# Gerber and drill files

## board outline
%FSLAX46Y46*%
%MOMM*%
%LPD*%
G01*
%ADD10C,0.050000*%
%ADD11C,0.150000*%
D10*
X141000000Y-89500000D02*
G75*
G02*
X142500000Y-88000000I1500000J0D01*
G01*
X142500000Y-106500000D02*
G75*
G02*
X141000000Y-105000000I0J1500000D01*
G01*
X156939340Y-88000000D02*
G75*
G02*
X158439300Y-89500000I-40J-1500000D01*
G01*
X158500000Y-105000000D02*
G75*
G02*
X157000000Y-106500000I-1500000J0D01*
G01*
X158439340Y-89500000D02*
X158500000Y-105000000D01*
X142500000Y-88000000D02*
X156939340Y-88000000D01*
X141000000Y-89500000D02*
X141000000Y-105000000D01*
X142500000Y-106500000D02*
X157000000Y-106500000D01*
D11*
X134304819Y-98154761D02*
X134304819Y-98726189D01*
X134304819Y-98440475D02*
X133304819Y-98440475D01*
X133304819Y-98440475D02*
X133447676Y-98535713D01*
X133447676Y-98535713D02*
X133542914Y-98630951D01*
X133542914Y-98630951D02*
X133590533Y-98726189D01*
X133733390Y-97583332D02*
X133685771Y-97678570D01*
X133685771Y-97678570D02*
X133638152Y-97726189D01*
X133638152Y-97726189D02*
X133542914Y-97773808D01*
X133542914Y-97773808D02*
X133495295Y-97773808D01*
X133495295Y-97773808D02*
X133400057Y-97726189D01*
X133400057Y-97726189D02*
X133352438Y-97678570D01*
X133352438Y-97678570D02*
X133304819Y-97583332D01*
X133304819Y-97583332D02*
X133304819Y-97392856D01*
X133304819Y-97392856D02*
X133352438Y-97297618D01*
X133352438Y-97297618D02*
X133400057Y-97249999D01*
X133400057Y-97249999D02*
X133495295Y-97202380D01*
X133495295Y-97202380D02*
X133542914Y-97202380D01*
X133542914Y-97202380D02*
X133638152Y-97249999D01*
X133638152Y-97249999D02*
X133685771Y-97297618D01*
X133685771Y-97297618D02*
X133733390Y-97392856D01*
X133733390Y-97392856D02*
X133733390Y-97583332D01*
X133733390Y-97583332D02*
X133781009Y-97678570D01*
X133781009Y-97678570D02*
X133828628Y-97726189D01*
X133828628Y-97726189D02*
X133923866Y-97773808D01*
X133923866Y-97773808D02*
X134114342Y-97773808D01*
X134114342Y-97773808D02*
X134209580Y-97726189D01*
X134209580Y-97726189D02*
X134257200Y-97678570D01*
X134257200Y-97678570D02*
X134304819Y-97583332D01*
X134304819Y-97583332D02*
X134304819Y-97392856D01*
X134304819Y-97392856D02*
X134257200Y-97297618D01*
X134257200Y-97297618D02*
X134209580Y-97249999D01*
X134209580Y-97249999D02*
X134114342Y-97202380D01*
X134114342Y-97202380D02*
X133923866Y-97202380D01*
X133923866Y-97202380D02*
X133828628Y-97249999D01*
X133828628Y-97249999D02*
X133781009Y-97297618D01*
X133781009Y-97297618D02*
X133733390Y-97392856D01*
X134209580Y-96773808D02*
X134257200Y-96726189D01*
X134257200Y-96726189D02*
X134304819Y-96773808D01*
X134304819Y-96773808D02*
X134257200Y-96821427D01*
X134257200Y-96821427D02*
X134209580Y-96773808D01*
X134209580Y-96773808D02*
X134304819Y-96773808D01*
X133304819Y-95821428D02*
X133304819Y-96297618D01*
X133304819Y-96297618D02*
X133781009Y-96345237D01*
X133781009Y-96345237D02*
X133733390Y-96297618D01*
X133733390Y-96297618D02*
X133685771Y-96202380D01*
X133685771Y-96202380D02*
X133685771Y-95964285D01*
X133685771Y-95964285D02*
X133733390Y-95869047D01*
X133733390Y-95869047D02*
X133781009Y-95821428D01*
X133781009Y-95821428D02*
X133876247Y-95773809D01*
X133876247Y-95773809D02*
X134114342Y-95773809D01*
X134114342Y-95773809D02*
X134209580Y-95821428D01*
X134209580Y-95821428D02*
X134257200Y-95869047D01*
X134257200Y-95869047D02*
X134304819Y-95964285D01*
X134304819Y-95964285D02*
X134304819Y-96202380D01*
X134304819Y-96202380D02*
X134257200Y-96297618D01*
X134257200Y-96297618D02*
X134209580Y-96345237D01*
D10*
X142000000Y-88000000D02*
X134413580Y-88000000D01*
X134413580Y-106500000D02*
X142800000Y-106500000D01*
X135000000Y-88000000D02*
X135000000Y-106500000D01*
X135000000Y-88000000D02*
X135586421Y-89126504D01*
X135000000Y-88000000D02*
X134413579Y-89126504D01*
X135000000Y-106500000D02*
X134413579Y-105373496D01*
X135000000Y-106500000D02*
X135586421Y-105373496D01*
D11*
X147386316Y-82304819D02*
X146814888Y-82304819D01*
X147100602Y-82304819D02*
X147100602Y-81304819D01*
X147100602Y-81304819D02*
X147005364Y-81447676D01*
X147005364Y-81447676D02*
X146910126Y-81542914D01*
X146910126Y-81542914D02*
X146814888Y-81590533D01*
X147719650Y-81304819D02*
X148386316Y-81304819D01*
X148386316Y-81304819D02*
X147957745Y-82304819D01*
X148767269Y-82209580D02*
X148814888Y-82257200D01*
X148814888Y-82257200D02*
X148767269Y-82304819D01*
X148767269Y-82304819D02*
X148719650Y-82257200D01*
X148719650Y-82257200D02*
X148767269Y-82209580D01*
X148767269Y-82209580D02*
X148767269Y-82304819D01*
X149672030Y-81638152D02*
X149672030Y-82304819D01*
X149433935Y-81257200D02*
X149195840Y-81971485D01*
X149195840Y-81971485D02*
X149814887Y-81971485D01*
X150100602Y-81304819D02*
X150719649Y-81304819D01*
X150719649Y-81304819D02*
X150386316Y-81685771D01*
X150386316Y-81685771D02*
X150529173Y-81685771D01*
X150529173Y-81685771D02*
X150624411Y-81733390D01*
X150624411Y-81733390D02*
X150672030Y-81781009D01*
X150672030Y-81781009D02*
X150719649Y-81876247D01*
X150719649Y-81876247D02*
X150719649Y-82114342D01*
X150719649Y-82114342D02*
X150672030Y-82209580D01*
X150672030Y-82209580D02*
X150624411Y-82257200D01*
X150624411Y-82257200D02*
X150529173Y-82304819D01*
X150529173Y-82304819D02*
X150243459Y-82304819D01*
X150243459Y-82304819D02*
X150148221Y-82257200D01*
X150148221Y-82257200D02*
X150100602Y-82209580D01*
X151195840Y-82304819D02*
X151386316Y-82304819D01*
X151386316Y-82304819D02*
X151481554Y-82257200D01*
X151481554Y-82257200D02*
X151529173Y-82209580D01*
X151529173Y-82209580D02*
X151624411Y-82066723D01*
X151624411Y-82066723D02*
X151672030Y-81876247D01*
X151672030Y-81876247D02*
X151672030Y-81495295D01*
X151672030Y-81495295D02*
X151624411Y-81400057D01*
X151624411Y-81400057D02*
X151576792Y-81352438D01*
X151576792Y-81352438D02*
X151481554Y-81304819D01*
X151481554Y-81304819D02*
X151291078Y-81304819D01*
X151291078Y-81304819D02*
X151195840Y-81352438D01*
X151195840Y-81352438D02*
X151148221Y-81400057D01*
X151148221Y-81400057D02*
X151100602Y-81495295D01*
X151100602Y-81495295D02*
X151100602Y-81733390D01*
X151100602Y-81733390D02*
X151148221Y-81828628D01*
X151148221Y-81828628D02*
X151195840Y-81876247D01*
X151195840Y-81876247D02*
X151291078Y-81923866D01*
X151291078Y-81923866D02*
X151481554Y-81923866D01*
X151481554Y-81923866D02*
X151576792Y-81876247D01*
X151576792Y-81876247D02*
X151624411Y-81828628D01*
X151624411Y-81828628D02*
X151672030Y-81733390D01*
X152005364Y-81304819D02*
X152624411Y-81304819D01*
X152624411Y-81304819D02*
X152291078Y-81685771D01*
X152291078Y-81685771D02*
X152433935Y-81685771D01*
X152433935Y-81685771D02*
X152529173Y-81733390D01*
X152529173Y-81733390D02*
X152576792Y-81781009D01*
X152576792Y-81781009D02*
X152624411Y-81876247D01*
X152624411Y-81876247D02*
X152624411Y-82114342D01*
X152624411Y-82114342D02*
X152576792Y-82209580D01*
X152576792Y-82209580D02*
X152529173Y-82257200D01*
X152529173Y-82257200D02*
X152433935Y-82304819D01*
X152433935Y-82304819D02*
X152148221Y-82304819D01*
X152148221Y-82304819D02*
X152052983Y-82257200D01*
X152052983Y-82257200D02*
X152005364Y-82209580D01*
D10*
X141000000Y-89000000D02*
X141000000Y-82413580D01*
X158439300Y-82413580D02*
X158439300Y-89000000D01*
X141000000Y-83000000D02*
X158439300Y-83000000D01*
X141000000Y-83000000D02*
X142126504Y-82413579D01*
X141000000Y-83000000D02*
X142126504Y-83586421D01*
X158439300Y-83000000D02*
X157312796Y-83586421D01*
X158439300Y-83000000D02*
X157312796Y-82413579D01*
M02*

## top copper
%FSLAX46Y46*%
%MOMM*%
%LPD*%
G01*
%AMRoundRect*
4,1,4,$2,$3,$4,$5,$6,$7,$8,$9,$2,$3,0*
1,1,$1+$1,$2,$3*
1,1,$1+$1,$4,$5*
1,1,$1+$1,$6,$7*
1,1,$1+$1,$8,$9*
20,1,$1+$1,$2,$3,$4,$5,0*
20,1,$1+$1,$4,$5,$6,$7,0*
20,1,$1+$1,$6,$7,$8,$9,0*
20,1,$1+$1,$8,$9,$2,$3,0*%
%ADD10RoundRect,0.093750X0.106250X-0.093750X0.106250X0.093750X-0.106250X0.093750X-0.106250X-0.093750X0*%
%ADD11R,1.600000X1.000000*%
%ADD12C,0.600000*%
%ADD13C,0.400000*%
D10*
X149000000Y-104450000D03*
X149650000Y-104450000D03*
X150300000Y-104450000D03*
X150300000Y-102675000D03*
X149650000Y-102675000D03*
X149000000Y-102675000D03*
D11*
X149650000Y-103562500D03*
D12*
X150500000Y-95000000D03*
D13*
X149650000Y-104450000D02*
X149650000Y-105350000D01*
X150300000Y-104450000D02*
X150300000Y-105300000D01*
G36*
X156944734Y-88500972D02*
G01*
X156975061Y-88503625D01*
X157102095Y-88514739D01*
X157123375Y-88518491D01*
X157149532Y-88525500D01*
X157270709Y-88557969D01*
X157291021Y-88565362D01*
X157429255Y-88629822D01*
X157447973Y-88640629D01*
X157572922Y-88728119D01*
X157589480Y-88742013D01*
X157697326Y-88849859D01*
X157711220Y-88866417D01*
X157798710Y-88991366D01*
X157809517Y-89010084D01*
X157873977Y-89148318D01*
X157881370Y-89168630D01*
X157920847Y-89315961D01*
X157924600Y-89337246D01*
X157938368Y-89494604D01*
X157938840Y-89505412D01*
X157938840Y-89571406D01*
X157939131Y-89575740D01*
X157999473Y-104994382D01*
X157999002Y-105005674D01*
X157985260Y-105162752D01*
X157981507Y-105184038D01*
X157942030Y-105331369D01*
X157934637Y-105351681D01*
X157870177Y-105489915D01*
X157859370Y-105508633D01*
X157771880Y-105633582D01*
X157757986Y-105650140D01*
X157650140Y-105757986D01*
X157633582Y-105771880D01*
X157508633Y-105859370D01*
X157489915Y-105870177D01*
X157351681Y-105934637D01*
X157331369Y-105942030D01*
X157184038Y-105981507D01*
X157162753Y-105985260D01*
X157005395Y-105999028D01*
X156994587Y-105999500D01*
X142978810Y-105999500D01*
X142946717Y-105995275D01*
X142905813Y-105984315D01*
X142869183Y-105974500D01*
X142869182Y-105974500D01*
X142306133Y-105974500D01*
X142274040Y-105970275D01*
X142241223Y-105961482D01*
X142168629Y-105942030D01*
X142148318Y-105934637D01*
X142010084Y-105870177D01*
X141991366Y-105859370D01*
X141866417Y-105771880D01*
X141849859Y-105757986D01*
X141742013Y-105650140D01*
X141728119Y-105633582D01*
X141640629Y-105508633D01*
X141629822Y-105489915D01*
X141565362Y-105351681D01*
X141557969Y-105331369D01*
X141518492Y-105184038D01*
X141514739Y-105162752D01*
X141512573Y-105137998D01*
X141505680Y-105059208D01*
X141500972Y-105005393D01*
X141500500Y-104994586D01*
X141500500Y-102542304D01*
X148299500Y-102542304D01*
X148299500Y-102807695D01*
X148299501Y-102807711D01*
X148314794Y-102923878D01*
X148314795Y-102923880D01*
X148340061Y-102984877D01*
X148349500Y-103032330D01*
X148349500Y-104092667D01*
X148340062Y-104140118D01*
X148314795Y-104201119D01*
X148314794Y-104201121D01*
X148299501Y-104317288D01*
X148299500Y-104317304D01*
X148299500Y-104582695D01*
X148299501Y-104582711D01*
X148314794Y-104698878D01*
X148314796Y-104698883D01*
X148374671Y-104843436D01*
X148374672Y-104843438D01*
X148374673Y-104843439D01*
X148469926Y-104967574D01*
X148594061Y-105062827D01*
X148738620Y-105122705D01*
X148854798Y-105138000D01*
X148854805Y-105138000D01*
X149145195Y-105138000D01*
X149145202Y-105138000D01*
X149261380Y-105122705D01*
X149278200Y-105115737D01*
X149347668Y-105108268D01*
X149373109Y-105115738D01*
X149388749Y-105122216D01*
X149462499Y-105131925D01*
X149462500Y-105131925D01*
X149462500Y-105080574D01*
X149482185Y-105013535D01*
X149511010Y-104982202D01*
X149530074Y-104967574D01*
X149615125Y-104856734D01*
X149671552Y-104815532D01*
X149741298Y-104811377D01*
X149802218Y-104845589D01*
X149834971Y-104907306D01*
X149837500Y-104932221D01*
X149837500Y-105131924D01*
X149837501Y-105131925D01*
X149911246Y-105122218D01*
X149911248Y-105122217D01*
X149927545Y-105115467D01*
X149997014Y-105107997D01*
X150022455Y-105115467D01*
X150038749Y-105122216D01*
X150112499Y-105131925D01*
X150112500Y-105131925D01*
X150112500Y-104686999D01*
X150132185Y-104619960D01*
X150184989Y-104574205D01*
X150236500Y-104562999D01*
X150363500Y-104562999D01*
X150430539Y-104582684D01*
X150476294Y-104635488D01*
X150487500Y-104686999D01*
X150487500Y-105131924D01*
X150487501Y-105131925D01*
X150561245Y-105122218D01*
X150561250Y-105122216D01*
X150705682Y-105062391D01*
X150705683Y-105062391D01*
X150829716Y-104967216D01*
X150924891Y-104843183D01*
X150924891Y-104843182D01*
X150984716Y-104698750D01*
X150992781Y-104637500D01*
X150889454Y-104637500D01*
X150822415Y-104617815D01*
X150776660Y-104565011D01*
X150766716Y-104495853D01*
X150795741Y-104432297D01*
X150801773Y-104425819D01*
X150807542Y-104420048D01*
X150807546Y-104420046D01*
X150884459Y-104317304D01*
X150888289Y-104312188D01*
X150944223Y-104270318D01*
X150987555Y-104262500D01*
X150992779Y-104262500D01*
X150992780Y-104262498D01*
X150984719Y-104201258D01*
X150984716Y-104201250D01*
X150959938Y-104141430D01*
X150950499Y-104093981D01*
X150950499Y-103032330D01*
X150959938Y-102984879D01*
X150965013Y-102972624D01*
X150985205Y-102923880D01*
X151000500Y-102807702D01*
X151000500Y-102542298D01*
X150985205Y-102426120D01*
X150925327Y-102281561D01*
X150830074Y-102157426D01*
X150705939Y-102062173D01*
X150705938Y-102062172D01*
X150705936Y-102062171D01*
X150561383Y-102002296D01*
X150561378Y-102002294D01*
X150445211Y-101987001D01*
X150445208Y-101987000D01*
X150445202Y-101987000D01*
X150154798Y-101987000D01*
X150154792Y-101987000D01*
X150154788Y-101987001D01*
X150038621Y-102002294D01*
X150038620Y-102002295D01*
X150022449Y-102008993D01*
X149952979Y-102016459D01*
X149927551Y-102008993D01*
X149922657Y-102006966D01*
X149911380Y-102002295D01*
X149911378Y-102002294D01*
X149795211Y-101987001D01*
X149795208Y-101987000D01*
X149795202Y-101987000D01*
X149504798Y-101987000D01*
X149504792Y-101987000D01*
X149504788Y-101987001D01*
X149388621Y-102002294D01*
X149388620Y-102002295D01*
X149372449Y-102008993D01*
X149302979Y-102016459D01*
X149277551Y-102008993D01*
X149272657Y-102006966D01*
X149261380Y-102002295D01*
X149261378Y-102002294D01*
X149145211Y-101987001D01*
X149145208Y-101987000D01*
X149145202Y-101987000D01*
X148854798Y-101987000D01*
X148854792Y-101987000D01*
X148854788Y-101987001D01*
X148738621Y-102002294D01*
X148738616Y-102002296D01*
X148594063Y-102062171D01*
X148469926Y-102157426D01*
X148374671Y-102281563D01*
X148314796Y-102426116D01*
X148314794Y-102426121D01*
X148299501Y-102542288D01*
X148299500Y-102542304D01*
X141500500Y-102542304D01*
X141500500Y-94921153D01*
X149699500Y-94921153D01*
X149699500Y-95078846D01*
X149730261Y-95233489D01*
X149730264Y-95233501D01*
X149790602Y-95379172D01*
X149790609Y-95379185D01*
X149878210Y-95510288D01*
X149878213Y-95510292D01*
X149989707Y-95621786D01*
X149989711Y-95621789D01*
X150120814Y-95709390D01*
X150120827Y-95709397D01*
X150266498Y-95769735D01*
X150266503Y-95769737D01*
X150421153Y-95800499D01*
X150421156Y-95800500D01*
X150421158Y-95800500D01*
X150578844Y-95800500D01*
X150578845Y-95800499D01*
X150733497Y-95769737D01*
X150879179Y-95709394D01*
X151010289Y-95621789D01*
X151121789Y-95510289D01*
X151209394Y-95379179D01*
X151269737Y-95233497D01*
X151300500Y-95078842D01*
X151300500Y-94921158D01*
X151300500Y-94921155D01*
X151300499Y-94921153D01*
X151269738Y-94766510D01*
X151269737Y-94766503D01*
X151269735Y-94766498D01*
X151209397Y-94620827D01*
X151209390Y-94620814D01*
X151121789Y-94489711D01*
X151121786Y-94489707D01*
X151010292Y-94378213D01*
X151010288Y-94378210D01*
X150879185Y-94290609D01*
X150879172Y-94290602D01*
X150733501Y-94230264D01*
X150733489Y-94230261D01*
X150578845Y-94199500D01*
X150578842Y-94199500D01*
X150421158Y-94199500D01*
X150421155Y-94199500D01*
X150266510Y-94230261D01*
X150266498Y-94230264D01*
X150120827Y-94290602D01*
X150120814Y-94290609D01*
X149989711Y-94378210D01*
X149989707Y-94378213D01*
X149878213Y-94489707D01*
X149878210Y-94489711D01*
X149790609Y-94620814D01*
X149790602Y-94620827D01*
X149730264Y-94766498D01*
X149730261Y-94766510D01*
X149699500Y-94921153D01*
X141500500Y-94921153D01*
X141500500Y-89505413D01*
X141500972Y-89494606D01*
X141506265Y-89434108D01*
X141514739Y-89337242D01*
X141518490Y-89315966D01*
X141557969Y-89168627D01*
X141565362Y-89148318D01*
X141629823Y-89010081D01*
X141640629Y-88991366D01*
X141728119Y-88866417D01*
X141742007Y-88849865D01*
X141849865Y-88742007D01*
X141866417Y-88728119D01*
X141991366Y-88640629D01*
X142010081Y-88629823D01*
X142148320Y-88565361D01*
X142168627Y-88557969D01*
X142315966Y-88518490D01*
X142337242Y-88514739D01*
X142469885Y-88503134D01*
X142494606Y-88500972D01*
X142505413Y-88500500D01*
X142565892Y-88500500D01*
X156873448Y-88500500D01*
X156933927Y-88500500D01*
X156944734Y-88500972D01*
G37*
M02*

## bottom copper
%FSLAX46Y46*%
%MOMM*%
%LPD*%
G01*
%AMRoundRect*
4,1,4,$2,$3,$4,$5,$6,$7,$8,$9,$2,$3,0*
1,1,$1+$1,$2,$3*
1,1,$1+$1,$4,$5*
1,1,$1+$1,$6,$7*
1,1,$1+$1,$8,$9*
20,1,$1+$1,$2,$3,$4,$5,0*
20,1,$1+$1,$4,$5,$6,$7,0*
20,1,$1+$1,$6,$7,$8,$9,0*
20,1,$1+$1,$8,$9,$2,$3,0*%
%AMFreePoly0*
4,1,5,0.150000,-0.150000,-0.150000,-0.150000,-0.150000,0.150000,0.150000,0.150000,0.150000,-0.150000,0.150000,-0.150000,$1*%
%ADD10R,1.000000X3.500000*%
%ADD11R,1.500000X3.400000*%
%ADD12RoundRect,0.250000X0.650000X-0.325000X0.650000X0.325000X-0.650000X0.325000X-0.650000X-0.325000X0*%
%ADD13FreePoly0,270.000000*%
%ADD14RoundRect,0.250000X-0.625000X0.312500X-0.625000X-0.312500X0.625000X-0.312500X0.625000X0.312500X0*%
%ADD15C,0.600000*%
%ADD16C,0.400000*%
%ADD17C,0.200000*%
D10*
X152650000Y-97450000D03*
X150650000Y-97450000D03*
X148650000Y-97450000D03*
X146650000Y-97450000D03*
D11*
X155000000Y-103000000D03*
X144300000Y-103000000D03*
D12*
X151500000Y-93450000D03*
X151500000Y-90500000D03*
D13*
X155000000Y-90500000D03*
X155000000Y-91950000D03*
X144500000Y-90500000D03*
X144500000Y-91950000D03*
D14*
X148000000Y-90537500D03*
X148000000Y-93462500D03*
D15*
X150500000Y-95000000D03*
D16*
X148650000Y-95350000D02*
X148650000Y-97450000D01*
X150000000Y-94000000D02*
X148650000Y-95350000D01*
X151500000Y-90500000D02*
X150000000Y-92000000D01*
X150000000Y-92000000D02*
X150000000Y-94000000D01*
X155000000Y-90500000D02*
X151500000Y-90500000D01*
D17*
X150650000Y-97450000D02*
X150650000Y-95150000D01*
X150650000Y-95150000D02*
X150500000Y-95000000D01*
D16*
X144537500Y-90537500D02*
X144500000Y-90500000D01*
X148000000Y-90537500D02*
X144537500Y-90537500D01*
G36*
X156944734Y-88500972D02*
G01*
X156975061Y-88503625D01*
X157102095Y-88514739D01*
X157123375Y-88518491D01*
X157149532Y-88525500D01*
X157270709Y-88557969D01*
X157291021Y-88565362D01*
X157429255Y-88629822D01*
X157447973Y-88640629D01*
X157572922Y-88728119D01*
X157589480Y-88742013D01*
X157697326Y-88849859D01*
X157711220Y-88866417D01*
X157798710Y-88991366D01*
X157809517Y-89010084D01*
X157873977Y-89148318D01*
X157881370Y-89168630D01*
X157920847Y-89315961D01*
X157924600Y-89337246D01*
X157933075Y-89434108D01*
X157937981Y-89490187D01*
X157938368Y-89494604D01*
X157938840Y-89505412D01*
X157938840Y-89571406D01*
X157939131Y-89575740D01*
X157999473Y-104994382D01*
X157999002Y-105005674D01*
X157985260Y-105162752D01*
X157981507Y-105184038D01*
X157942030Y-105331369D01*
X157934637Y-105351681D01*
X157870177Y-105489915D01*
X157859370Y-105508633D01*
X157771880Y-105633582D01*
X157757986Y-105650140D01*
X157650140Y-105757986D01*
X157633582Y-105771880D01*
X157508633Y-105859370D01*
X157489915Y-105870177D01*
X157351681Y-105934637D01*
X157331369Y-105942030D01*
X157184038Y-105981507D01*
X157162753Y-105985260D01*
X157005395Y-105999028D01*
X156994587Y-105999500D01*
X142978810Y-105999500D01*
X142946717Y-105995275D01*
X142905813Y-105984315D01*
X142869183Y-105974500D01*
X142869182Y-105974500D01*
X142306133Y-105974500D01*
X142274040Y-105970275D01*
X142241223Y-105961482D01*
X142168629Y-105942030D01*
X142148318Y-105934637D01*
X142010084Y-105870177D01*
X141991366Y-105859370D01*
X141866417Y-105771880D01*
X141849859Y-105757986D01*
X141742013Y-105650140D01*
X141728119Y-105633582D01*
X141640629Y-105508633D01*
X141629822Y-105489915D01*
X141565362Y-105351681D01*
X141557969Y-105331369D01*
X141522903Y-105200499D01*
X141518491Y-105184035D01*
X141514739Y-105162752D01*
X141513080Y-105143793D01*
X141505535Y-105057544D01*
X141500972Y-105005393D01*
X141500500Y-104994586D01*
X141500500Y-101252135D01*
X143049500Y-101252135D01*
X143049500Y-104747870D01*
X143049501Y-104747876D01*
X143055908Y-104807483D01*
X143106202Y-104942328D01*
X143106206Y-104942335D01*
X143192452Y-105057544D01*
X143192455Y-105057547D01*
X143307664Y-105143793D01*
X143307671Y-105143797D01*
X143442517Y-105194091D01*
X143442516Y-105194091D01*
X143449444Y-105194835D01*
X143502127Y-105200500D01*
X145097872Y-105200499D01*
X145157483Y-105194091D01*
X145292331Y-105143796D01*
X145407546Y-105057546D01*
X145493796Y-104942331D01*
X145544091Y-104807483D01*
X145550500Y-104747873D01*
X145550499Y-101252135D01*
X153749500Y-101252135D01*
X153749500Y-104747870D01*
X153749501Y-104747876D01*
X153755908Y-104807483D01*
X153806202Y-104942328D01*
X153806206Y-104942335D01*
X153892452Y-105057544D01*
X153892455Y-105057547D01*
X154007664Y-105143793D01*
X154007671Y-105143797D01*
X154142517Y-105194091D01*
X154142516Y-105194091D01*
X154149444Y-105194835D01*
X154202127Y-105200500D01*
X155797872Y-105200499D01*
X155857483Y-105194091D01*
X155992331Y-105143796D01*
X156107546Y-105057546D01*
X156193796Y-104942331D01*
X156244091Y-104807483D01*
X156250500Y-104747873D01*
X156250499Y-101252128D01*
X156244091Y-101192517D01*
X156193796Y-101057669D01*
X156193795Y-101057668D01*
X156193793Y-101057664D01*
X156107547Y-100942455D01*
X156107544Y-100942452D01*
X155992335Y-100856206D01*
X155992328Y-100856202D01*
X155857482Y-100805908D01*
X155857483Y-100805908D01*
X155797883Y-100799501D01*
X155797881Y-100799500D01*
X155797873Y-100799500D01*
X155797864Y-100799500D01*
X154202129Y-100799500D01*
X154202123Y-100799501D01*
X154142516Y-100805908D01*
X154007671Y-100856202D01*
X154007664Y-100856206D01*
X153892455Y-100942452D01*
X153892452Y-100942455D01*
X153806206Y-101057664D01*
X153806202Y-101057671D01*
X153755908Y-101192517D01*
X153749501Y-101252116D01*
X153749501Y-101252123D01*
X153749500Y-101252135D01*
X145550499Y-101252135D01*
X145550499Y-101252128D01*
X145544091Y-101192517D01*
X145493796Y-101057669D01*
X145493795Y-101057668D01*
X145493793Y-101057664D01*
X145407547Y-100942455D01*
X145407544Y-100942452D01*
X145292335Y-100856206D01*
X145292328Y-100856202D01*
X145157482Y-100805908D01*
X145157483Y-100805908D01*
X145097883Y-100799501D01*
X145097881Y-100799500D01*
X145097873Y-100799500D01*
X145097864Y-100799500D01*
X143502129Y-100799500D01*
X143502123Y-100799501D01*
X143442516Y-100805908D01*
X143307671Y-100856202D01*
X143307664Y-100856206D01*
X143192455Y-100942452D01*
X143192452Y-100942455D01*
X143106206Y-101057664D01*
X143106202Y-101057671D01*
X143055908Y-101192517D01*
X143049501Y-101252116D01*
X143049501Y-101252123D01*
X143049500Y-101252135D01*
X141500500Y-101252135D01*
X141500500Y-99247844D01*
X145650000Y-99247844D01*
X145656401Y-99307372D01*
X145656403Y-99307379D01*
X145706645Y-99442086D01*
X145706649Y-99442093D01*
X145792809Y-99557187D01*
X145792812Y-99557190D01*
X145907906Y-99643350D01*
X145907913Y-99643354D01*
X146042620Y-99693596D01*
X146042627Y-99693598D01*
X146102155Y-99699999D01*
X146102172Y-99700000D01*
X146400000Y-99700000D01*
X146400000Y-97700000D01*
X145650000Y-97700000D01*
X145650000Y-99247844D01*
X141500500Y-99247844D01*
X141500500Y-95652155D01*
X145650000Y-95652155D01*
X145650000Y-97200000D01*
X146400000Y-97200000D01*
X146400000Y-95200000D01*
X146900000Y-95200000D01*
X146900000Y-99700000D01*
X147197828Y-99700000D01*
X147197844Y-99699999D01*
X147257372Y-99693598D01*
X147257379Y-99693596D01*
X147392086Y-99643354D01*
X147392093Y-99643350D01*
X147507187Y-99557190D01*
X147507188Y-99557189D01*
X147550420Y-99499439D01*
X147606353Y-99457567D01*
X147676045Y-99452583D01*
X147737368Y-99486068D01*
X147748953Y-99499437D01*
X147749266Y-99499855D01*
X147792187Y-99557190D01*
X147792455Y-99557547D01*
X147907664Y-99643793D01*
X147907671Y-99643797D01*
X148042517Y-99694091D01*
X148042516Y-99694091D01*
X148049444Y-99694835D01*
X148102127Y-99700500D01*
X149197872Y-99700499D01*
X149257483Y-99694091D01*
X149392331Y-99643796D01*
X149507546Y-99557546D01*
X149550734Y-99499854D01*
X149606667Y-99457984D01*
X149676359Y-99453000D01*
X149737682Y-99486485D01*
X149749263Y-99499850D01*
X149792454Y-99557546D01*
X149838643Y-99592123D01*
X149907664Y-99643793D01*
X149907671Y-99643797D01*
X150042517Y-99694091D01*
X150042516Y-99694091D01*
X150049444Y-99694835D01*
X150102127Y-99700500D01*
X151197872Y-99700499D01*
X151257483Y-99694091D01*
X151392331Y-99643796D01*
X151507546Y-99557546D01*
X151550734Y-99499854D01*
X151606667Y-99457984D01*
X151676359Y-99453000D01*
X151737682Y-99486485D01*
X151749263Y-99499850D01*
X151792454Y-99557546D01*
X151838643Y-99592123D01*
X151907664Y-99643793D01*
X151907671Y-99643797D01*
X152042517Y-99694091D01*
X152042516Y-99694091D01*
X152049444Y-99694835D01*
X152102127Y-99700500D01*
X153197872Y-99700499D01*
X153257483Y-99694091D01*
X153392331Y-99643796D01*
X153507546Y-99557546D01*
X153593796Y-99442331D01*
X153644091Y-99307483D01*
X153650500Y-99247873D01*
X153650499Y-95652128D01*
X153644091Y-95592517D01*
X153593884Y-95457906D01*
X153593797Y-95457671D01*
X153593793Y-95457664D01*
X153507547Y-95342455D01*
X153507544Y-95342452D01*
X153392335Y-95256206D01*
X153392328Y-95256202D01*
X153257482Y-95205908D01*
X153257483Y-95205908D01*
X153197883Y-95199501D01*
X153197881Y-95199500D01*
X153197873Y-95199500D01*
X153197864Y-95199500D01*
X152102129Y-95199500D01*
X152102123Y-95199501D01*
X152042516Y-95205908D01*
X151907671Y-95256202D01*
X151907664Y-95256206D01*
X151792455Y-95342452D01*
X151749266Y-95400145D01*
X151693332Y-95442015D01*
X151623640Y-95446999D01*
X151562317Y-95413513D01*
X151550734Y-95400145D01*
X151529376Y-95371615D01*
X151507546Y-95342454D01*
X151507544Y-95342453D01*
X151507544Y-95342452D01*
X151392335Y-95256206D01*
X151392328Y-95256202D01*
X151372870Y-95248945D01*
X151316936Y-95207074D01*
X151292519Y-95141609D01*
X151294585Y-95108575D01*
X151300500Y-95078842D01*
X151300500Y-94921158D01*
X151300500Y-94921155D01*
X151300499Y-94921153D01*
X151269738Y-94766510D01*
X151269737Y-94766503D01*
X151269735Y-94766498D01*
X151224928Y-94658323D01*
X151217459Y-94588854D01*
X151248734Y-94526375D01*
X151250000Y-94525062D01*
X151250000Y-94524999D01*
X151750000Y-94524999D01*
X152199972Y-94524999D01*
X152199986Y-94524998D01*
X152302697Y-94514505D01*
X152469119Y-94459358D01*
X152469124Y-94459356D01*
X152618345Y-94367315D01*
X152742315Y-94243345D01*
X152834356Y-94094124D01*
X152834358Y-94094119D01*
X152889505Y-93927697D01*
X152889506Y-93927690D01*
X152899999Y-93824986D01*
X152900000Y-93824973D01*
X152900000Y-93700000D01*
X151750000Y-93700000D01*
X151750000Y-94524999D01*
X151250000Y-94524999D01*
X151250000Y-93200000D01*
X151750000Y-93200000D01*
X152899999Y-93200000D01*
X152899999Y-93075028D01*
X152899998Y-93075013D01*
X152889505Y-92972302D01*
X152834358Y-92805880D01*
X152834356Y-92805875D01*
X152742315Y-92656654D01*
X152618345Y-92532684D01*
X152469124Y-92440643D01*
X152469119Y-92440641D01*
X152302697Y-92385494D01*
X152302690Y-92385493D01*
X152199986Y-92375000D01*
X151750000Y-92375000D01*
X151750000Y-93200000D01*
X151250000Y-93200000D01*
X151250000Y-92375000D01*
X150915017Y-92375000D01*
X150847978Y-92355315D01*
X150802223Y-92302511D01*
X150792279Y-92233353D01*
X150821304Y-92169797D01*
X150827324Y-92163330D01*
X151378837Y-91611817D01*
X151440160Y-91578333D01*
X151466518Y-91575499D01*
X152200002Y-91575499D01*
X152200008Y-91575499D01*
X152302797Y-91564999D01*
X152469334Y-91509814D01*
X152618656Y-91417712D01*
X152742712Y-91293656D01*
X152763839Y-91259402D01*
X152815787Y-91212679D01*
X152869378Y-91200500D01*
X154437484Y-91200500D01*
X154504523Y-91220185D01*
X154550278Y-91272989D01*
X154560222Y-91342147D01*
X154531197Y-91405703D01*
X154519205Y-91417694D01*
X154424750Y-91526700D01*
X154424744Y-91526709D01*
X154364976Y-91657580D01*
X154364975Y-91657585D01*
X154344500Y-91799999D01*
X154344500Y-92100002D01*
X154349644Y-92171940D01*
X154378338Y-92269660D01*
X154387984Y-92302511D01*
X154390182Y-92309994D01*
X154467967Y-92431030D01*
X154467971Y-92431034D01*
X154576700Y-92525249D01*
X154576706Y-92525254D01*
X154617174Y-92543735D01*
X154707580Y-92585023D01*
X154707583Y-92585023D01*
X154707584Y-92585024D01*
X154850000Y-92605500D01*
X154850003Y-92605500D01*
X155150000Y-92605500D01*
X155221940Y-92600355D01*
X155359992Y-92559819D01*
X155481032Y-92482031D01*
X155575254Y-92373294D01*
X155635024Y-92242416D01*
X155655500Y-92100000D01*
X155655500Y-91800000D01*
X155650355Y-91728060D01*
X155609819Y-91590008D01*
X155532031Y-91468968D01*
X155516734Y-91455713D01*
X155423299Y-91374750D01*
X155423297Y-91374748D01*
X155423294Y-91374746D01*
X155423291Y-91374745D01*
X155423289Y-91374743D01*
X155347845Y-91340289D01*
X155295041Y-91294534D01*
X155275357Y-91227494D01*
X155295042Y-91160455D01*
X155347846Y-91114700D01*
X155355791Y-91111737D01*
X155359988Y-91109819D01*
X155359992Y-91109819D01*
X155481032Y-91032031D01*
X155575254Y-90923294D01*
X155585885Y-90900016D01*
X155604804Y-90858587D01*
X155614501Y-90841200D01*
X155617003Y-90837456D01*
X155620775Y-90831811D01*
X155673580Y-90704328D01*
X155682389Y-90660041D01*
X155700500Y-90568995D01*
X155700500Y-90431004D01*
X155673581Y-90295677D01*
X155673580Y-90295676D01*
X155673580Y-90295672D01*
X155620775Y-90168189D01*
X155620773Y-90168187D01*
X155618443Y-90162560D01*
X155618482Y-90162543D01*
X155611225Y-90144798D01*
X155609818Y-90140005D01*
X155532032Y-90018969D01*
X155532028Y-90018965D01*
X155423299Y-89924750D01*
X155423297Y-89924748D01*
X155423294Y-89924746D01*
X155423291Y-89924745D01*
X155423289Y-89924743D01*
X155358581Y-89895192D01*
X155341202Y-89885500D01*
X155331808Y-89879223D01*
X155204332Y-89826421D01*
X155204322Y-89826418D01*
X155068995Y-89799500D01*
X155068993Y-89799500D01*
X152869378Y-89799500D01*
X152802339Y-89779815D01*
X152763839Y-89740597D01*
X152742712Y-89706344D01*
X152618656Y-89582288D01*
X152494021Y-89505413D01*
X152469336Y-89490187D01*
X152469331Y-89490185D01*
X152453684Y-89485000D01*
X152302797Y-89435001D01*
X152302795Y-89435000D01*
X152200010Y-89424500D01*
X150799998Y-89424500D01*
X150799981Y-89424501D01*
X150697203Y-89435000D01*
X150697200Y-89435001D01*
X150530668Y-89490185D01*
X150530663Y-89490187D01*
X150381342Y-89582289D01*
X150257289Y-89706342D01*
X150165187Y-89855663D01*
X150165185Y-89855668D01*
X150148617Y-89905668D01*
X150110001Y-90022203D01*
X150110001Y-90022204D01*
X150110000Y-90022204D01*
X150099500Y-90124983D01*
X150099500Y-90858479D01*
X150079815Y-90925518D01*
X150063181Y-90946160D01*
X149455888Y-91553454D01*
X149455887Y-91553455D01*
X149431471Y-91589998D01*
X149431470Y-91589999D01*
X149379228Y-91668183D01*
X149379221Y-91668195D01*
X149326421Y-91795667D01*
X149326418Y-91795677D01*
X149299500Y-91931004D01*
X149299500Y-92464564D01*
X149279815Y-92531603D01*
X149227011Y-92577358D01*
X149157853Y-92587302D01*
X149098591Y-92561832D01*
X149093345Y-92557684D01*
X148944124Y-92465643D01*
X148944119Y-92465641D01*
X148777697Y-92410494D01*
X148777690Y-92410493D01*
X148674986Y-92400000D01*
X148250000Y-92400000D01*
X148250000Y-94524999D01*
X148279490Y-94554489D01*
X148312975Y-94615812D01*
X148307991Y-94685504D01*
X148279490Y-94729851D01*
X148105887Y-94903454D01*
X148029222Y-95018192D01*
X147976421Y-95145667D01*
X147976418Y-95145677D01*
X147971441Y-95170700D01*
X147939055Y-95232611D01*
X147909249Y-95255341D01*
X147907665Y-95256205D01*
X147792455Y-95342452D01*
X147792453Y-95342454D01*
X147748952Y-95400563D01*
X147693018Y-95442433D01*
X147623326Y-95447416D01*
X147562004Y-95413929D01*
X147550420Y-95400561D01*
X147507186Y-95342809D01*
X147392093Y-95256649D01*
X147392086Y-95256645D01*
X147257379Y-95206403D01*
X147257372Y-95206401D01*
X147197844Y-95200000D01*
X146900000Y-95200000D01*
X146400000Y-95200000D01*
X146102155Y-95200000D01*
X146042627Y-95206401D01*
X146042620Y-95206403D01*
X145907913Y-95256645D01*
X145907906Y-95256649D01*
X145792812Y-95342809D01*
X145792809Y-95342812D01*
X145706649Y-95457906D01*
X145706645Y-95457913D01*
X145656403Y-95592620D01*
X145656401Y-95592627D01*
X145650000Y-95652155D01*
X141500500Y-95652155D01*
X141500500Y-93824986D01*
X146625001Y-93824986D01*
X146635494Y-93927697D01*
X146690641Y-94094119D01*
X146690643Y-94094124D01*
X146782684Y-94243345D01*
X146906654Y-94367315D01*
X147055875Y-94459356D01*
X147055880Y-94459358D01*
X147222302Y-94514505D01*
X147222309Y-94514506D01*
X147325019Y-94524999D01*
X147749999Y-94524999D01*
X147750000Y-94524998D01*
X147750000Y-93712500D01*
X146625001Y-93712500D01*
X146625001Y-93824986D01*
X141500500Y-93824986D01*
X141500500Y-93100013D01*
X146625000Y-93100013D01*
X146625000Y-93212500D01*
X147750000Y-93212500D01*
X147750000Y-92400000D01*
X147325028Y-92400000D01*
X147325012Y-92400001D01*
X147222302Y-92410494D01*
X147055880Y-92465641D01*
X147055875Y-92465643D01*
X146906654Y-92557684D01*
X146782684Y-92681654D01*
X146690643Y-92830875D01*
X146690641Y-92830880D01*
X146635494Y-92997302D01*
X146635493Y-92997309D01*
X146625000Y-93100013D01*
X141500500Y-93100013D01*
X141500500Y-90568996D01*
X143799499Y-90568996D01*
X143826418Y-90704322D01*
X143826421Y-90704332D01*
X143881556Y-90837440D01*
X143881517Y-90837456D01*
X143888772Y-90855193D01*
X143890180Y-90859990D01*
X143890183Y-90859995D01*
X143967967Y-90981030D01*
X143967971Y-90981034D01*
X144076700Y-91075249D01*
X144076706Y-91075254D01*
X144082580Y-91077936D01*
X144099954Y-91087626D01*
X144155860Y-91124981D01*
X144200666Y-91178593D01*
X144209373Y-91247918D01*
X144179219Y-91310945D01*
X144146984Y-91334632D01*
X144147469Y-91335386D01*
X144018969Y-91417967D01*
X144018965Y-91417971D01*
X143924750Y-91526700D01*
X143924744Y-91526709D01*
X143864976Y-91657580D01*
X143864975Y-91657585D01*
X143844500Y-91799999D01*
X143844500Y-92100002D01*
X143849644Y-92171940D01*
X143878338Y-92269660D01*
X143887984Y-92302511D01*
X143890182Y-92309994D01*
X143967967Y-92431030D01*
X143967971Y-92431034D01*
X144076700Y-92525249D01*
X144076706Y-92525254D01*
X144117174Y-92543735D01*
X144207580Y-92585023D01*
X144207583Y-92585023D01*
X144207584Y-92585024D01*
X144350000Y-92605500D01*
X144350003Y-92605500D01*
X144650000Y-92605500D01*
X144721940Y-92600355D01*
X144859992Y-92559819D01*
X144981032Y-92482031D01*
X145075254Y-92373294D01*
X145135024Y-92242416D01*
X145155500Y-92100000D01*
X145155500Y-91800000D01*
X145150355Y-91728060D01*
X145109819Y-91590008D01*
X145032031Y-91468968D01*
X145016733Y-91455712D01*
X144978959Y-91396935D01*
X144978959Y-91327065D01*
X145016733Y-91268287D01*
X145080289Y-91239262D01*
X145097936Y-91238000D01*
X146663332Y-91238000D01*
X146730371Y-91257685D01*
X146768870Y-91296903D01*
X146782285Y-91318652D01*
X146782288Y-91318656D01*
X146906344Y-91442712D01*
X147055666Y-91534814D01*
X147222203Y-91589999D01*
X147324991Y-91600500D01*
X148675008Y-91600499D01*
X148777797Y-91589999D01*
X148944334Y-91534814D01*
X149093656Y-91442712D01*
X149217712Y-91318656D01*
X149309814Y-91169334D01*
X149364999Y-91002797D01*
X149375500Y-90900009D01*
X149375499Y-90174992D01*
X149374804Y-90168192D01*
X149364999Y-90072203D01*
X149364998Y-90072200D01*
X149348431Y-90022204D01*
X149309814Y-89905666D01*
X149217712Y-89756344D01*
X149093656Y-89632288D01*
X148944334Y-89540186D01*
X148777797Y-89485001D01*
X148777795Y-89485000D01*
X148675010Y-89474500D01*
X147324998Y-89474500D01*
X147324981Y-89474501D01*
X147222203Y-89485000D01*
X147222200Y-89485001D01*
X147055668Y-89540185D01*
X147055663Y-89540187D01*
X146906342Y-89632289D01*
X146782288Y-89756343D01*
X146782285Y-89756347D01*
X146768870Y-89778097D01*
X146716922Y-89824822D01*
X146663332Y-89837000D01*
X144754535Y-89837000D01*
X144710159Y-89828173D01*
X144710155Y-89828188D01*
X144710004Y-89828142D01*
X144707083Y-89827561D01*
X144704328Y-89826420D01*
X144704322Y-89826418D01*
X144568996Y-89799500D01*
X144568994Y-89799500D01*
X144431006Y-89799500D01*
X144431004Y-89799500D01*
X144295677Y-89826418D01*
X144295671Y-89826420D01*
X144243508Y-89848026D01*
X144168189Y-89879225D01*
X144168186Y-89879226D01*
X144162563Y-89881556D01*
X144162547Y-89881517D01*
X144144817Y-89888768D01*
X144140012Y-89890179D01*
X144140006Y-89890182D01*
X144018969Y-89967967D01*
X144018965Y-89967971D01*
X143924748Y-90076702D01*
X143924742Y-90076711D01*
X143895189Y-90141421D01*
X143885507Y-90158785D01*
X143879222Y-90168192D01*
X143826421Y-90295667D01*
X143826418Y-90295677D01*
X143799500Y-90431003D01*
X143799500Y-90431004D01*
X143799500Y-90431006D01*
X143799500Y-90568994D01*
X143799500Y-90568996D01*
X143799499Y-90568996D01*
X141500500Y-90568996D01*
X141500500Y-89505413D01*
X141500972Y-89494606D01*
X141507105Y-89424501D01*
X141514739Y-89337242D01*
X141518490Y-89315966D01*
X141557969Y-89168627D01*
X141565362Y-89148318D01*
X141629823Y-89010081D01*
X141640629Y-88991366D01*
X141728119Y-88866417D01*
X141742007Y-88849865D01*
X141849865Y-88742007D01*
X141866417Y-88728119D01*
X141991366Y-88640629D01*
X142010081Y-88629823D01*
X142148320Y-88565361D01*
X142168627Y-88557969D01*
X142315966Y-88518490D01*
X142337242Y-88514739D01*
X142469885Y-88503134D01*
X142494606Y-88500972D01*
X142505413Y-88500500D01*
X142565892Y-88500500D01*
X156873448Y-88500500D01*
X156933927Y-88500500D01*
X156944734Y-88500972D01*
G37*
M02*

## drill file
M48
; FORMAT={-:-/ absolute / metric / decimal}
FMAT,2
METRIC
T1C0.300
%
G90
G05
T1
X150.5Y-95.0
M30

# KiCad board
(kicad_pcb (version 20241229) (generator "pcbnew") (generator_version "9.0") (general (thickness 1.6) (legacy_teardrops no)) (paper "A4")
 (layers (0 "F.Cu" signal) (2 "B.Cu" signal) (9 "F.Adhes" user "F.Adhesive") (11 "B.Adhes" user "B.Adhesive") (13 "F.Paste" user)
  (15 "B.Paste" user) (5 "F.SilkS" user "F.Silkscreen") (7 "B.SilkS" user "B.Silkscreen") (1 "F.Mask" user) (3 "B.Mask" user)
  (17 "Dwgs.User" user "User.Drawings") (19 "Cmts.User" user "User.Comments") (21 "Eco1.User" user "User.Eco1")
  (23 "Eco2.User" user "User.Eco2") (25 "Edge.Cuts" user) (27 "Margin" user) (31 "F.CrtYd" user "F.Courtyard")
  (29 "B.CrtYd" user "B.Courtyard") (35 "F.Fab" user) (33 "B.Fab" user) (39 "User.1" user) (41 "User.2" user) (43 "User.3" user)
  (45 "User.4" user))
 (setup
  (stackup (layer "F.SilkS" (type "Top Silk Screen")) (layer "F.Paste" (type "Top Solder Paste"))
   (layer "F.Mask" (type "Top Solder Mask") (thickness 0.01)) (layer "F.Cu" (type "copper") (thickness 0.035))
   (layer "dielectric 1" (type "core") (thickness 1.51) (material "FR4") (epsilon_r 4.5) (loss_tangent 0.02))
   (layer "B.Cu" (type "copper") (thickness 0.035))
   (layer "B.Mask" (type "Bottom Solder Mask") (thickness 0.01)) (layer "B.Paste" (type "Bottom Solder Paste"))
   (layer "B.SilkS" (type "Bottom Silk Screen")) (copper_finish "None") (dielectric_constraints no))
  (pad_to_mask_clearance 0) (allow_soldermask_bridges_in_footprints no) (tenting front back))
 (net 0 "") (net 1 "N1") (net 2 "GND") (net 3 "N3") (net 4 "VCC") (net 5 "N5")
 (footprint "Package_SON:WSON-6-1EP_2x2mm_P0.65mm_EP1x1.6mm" (layer "F.Cu") (at 149.65 103.5625 90)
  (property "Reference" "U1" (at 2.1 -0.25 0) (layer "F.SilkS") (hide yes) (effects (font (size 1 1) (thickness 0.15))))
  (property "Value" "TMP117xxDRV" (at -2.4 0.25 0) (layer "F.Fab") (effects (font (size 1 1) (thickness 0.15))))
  (pad "" smd roundrect (at 0 -0.4 90) (size 0.81 0.64) (layers "F.Paste") (roundrect_rratio 0.25))
  (pad "" smd roundrect (at 0 0.4 90) (size 0.81 0.64) (layers "F.Paste") (roundrect_rratio 0.25))
  (pad "1" smd roundrect (at -0.8875 -0.65 90) (size 0.375 0.4) (layers "F.Cu" "F.Mask" "F.Paste") (roundrect_rratio 0.25) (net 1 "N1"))
  (pad "2" smd roundrect (at -0.8875 0 90) (size 0.375 0.4) (layers "F.Cu" "F.Mask" "F.Paste") (roundrect_rratio 0.25) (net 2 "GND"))
  (pad "3" smd roundrect (at -0.8875 0.65 90) (size 0.375 0.4) (layers "F.Cu" "F.Mask" "F.Paste") (roundrect_rratio 0.25) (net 2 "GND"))
  (pad "4" smd roundrect (at 0.8875 0.65 90) (size 0.375 0.4) (layers "F.Cu" "F.Mask" "F.Paste") (roundrect_rratio 0.25) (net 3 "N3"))
  (pad "5" smd roundrect (at 0.8875 0 90) (size 0.375 0.4) (layers "F.Cu" "F.Mask" "F.Paste") (roundrect_rratio 0.25) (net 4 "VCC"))
  (pad "6" smd roundrect (at 0.8875 -0.65 90) (size 0.375 0.4) (layers "F.Cu" "F.Mask" "F.Paste") (roundrect_rratio 0.25) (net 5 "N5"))
  (pad "7" smd rect (at 0 0 90) (size 1 1.6) (layers "F.Cu" "F.Mask") (zone_connect 2)))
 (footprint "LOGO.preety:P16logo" (layer "F.Cu") (at 144.5 99.5)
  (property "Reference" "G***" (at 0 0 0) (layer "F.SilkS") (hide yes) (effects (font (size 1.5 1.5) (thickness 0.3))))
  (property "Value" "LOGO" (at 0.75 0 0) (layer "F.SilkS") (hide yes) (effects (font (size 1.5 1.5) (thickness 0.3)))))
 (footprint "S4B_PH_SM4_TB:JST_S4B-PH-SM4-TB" (layer "B.Cu") (at 149.65 100.2 180)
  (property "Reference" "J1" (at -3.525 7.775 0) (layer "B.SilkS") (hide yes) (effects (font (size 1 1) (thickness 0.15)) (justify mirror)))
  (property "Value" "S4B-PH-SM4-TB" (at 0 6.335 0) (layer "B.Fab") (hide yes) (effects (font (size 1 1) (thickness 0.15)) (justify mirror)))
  (pad "1" smd rect (at -3 2.75 180) (size 1 3.5) (layers "B.Cu" "B.Mask" "B.Paste") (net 1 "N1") (solder_mask_margin 0.102))
  (pad "2" smd rect (at -1 2.75 180) (size 1 3.5) (layers "B.Cu" "B.Mask" "B.Paste") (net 5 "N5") (solder_mask_margin 0.102))
  (pad "3" smd rect (at 1 2.75 180) (size 1 3.5) (layers "B.Cu" "B.Mask" "B.Paste") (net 4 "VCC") (solder_mask_margin 0.102))
  (pad "4" smd rect (at 3 2.75 180) (size 1 3.5) (layers "B.Cu" "B.Mask" "B.Paste") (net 2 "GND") (solder_mask_margin 0.102))
  (pad "SH1" smd rect (at -5.35 -2.8 180) (size 1.5 3.4) (layers "B.Cu" "B.Mask" "B.Paste") (solder_mask_margin 0.102))
  (pad "SH2" smd rect (at 5.35 -2.8 180) (size 1.5 3.4) (layers "B.Cu" "B.Mask" "B.Paste") (solder_mask_margin 0.102)))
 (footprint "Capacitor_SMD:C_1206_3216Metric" (layer "B.Cu") (at 151.5 91.975 90)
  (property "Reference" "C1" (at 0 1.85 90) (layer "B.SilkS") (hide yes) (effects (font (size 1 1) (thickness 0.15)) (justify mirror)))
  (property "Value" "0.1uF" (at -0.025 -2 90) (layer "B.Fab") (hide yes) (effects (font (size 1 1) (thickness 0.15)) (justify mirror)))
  (pad "1" smd roundrect (at -1.475 0 90) (size 1.15 1.8) (layers "B.Cu" "B.Mask" "B.Paste") (roundrect_rratio 0.217391) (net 2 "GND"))
  (pad "2" smd roundrect (at 1.475 0 90) (size 1.15 1.8) (layers "B.Cu" "B.Mask" "B.Paste") (roundrect_rratio 0.217391) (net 4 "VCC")))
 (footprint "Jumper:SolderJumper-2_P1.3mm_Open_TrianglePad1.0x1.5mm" (layer "B.Cu") (at 155 91.225 -90)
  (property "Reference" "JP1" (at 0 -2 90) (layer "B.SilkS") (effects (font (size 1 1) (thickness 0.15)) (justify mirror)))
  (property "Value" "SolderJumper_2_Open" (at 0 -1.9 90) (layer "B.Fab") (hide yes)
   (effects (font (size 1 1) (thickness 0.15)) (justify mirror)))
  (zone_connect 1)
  (pad "1" smd custom (at -0.725 0 270) (size 0.3 0.3) (layers "B.Cu" "B.Mask") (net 4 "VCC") (zone_connect 2) (thermal_bridge_angle 45)
   (options (clearance outline) (anchor rect)) (primitives))
  (pad "2" smd custom (at 0.725 0 270) (size 0.3 0.3) (layers "B.Cu" "B.Mask") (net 3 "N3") (zone_connect 2) (thermal_bridge_angle 45)
   (options (clearance outline) (anchor rect)) (primitives)))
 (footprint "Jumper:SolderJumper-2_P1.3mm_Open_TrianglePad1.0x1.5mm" (layer "B.Cu") (at 144.5 91.225 -90)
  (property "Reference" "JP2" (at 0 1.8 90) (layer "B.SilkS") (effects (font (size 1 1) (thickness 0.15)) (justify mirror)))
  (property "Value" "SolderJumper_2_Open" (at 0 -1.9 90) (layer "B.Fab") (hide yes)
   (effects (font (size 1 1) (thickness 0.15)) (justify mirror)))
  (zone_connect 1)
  (pad "1" smd custom (at -0.725 0 270) (size 0.3 0.3) (layers "B.Cu" "B.Mask") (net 3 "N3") (zone_connect 2) (thermal_bridge_angle 45)
   (options (clearance outline) (anchor rect)) (primitives))
  (pad "2" smd custom (at 0.725 0 270) (size 0.3 0.3) (layers "B.Cu" "B.Mask") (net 5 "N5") (zone_connect 2) (thermal_bridge_angle 45)
   (options (clearance outline) (anchor rect)) (primitives)))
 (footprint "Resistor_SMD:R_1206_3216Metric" (layer "B.Cu") (at 148 92 -90)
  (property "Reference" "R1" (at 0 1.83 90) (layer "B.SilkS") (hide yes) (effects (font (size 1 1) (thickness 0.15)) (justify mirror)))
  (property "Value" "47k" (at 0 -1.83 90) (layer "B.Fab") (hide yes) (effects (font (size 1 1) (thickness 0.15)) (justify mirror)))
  (pad "1" smd roundrect (at -1.4625 0 270) (size 1.125 1.75) (layers "B.Cu" "B.Mask" "B.Paste") (roundrect_rratio 0.222222) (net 3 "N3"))
  (pad "2" smd roundrect (at 1.4625 0 270) (size 1.125 1.75) (layers "B.Cu" "B.Mask" "B.Paste") (roundrect_rratio 0.222222) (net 2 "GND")))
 (gr_arc (start 141 89.5) (mid 141.43934 88.43934) (end 142.5 88) (stroke (width 0.05) (type default)) (layer "Edge.Cuts"))
 (gr_arc (start 142.5 106.5) (mid 141.43934 106.06066) (end 141 105) (stroke (width 0.05) (type default)) (layer "Edge.Cuts"))
 (gr_arc (start 156.93934 88) (mid 158 88.43934) (end 158.43934 89.5) (stroke (width 0.05) (type default)) (layer "Edge.Cuts"))
 (gr_arc (start 158.5 105) (mid 158.06066 106.06066) (end 157 106.5) (stroke (width 0.05) (type default)) (layer "Edge.Cuts"))
 (gr_line (start 158.43934 89.5) (end 158.5 105) (stroke (width 0.05) (type default)) (layer "Edge.Cuts"))
 (gr_line (start 142.5 88) (end 156.93934 88) (stroke (width 0.05) (type default)) (layer "Edge.Cuts"))
 (gr_line (start 141 89.5) (end 141 105) (stroke (width 0.05) (type default)) (layer "Edge.Cuts"))
 (gr_line (start 142.5 106.5) (end 157 106.5) (stroke (width 0.05) (type default)) (layer "Edge.Cuts"))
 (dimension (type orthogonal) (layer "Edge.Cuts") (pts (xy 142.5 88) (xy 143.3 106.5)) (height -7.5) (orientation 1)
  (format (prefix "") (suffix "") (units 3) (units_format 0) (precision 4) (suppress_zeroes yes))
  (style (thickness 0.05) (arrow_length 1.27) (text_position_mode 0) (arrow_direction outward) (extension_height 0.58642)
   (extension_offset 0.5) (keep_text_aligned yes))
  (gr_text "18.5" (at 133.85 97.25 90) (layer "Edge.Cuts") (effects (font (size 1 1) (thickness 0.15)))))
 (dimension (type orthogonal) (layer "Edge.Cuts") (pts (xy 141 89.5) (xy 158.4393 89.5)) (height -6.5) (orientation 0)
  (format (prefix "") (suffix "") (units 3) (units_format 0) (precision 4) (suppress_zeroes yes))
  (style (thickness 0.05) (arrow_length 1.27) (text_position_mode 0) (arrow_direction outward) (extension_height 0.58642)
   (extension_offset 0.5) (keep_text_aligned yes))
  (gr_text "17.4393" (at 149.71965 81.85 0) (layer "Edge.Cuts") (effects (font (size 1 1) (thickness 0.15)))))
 (segment (start 149.65 104.45) (end 149.65 105.35) (width 0.4) (layer "F.Cu") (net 2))
 (segment (start 150.3 104.45) (end 150.3 105.3) (width 0.4) (layer "F.Cu") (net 2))
 (segment (start 148.65 95.35) (end 148.65 97.45) (width 0.4) (layer "B.Cu") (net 4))
 (segment (start 150 94) (end 148.65 95.35) (width 0.4) (layer "B.Cu") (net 4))
 (segment (start 151.5 90.5) (end 150 92) (width 0.4) (layer "B.Cu") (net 4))
 (segment (start 150 92) (end 150 94) (width 0.4) (layer "B.Cu") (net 4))
 (segment (start 155 90.5) (end 151.5 90.5) (width 0.4) (layer "B.Cu") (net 4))
 (via (at 150.5 95) (size 0.6) (drill 0.3) (layers "F.Cu" "B.Cu") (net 5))
 (segment (start 150.65 97.45) (end 150.65 95.15) (width 0.2) (layer "B.Cu") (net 5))
 (segment (start 150.65 95.15) (end 150.5 95) (width 0.2) (layer "B.Cu") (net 5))
 (segment (start 144.5375 90.5375) (end 144.5 90.5) (width 0.4) (layer "B.Cu") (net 3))
 (segment (start 148 90.5375) (end 144.5375 90.5375) (width 0.4) (layer "B.Cu") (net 3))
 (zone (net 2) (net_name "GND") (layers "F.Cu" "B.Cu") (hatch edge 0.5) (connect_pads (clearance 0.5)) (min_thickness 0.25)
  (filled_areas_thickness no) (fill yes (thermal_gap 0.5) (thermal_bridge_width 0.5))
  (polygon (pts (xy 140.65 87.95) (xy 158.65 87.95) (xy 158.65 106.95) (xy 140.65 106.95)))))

